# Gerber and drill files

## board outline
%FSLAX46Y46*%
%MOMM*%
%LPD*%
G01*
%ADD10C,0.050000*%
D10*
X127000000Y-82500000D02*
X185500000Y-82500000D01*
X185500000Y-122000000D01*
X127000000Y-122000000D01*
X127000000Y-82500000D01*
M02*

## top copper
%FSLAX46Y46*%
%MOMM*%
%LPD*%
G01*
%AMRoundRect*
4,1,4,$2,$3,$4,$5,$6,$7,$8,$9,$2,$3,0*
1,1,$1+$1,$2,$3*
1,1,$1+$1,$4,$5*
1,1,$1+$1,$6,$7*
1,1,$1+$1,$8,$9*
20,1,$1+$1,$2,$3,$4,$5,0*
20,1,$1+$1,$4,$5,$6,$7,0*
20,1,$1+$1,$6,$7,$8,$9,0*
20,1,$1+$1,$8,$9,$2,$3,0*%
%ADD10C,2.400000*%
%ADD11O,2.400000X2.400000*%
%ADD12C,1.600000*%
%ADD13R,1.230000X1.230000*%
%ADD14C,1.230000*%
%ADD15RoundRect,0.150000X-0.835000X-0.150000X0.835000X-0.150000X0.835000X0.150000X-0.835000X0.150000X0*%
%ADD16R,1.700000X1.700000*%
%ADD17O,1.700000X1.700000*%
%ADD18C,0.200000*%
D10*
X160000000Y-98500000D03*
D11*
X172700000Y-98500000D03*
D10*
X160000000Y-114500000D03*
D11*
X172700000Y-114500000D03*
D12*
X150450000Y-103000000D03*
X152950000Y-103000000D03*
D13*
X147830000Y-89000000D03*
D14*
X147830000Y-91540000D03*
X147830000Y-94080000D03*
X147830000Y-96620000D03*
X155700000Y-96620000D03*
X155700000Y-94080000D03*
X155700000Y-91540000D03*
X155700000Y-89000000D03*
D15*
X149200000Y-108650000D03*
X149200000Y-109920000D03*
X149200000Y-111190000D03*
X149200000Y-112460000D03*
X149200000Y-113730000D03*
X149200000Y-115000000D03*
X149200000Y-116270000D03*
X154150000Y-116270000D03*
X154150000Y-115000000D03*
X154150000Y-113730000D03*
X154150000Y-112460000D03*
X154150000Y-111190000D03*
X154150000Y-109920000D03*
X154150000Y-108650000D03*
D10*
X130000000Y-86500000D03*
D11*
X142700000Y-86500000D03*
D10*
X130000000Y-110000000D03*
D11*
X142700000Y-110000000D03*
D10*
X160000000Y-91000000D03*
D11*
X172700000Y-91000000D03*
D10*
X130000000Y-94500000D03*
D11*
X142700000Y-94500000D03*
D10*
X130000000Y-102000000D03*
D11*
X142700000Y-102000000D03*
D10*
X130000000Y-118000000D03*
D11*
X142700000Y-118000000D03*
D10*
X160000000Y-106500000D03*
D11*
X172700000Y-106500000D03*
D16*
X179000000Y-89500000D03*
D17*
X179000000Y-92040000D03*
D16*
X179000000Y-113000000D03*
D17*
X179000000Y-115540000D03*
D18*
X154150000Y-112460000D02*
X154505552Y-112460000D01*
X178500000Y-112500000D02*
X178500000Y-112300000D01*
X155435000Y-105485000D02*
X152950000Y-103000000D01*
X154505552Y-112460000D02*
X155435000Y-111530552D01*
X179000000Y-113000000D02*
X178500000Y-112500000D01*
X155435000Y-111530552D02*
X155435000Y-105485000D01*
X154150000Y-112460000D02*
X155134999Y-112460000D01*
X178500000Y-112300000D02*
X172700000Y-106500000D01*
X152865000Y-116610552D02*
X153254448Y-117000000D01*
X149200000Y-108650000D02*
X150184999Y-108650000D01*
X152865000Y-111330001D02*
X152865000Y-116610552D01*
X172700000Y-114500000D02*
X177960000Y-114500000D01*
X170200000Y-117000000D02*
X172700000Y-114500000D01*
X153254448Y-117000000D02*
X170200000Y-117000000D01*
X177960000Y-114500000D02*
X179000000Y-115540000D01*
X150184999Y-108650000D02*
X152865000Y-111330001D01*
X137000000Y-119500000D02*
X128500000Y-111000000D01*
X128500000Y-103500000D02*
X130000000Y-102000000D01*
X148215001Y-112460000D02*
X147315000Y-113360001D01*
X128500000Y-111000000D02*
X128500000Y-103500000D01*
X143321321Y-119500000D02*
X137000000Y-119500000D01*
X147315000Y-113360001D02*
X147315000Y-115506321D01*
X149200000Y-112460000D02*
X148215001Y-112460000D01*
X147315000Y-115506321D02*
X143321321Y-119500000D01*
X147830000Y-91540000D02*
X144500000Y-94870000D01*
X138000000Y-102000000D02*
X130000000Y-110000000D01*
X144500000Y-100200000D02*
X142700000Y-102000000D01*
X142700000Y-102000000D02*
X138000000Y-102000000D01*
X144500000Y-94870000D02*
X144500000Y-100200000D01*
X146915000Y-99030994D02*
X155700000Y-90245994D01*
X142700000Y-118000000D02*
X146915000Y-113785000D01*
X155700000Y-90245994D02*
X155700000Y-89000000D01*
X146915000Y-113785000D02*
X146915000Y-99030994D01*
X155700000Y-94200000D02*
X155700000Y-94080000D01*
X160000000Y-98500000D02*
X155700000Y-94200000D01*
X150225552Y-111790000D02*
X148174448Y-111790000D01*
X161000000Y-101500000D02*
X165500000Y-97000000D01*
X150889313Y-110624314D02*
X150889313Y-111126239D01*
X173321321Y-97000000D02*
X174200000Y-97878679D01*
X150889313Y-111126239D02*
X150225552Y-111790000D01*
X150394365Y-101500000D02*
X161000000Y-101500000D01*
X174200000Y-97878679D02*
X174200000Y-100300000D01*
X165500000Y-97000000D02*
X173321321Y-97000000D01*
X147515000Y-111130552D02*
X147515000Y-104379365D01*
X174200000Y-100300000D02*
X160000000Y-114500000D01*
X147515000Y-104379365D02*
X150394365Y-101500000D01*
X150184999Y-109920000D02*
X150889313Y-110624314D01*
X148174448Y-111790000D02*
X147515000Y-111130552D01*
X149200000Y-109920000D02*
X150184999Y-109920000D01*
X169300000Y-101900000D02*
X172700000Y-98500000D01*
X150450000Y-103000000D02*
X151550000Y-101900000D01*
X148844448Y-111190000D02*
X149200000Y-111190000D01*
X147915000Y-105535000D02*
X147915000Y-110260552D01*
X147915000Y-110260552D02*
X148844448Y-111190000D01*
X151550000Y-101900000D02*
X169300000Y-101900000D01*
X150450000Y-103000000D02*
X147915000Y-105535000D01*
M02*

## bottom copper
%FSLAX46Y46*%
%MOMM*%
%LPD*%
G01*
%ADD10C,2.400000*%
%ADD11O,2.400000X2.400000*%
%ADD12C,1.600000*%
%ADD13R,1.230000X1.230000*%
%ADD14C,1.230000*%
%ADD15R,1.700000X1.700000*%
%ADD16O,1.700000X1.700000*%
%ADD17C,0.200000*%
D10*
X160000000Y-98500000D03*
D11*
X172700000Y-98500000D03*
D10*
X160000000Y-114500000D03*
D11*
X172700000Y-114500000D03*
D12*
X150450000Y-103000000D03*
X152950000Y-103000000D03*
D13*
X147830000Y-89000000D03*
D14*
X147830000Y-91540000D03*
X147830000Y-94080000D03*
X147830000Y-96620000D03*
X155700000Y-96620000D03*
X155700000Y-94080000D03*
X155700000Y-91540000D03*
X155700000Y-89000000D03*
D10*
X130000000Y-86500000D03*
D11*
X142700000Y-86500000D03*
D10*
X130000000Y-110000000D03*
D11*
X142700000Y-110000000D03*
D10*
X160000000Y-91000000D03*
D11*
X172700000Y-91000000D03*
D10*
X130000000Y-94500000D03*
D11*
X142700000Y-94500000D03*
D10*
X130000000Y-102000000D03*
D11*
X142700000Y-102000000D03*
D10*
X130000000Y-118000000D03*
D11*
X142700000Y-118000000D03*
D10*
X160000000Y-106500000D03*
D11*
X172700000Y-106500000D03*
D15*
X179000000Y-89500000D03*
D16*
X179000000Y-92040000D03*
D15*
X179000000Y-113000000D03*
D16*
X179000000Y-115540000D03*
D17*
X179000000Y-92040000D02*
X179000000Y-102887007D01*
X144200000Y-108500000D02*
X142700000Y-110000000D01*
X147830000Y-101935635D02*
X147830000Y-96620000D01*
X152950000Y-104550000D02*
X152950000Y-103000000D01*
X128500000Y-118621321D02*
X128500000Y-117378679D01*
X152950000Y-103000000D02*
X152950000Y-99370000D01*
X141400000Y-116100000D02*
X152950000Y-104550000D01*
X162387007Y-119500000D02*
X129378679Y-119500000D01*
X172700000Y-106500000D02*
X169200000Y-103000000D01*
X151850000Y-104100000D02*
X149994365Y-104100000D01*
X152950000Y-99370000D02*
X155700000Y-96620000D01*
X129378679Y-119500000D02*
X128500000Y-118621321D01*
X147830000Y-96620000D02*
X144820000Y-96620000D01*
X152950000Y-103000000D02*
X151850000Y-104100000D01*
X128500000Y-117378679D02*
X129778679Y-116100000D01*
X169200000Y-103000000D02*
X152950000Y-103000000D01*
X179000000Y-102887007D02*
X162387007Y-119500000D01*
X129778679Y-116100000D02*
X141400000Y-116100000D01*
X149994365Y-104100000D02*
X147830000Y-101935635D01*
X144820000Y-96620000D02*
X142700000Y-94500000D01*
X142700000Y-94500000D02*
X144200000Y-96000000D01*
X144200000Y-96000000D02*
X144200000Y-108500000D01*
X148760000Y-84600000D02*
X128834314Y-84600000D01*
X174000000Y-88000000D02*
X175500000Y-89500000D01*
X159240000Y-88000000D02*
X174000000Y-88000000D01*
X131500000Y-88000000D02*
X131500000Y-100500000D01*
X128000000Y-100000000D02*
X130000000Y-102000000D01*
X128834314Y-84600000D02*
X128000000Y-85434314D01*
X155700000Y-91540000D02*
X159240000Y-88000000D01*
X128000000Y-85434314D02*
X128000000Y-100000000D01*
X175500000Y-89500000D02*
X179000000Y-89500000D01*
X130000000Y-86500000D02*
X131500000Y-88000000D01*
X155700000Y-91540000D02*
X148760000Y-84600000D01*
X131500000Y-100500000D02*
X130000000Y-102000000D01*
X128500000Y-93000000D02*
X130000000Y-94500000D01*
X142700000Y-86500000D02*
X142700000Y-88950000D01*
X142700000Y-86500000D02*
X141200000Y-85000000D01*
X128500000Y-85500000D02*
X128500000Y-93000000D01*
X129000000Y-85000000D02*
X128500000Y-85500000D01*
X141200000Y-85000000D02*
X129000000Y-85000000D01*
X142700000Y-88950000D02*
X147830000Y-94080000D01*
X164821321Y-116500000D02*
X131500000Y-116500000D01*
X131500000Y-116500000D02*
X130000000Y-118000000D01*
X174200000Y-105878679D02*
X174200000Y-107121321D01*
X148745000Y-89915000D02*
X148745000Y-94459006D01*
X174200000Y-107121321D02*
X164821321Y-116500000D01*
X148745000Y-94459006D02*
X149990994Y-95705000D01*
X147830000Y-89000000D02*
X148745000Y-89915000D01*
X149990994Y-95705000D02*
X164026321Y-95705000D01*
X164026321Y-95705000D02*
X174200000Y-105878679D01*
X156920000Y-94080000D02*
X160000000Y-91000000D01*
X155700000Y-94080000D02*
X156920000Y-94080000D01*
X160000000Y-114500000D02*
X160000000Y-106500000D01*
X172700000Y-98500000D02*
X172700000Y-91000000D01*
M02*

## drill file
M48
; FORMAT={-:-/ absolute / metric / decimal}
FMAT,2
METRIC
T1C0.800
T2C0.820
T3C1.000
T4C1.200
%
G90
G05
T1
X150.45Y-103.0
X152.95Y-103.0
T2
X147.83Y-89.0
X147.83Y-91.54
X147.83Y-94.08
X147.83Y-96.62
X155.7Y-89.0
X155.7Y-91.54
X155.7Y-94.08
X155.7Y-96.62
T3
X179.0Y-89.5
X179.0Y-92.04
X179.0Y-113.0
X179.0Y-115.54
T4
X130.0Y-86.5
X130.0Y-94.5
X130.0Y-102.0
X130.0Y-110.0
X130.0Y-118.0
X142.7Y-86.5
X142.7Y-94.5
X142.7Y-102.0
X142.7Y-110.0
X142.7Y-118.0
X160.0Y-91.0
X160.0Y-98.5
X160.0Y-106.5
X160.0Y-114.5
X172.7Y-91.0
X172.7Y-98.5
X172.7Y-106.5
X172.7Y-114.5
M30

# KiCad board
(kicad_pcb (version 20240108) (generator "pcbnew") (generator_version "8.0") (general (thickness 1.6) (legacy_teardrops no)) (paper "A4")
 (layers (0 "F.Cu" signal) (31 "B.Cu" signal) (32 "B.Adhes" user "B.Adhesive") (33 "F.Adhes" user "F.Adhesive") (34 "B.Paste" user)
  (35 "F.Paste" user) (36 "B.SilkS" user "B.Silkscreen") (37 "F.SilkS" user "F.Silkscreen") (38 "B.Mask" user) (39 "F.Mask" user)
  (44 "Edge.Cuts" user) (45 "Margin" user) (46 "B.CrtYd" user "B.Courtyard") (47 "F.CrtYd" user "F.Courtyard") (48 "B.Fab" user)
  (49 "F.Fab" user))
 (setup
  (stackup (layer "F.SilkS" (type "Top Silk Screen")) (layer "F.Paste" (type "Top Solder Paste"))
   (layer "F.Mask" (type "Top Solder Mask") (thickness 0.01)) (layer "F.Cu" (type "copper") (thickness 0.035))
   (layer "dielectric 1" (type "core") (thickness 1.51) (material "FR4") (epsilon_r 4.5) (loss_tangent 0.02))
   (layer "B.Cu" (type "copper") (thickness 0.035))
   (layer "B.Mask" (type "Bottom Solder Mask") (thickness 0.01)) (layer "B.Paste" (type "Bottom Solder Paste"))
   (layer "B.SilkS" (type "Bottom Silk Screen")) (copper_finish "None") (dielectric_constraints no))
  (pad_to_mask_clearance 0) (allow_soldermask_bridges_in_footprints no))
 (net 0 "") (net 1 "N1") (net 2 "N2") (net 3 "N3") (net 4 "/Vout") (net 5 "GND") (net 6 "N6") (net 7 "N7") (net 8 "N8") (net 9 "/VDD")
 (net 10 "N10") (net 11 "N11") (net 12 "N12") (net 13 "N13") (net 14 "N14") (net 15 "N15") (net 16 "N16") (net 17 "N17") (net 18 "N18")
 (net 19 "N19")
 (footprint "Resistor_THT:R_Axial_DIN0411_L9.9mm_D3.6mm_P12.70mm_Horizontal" (layer "F.Cu") (at 160 98.5)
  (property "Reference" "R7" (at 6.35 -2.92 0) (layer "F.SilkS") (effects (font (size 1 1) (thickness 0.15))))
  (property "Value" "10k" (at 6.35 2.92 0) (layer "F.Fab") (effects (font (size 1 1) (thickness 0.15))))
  (pad "1" thru_hole circle (at 0 0) (size 2.4 2.4) (drill 1.2) (layers "*.Cu" "*.Mask") (remove_unused_layers no) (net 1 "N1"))
  (pad "2" thru_hole oval (at 12.7 0) (size 2.4 2.4) (drill 1.2) (layers "*.Cu" "*.Mask") (remove_unused_layers no) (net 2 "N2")))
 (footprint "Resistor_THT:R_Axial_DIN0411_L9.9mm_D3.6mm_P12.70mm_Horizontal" (layer "F.Cu") (at 160 114.5)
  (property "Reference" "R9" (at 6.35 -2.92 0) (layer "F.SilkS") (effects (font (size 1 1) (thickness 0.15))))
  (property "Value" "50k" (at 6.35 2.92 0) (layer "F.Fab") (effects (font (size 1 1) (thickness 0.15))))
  (pad "1" thru_hole circle (at 0 0) (size 2.4 2.4) (drill 1.2) (layers "*.Cu" "*.Mask") (remove_unused_layers no) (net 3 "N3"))
  (pad "2" thru_hole oval (at 12.7 0) (size 2.4 2.4) (drill 1.2) (layers "*.Cu" "*.Mask") (remove_unused_layers no) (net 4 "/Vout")))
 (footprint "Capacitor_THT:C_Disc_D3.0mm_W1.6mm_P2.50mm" (layer "F.Cu") (at 150.45 103)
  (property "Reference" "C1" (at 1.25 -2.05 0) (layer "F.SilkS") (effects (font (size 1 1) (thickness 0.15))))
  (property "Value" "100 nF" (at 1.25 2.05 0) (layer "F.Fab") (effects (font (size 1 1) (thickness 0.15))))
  (pad "1" thru_hole circle (at 0 0) (size 1.6 1.6) (drill 0.8) (layers "*.Cu" "*.Mask") (remove_unused_layers no) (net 2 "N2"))
  (pad "2" thru_hole circle (at 2.5 0) (size 1.6 1.6) (drill 0.8) (layers "*.Cu" "*.Mask") (remove_unused_layers no) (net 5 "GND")))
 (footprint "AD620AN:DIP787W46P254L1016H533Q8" (layer "F.Cu") (at 151.765 92.81)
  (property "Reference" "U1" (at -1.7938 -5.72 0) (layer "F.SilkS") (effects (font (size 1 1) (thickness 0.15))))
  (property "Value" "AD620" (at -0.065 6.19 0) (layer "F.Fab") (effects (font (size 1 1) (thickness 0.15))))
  (pad "1" thru_hole rect (at -3.935 -3.81) (size 1.23 1.23) (drill 0.82) (layers "*.Cu" "*.Mask") (remove_unused_layers no) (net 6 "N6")
   (solder_mask_margin 0.102))
  (pad "2" thru_hole circle (at -3.935 -1.27) (size 1.23 1.23) (drill 0.82) (layers "*.Cu" "*.Mask") (remove_unused_layers no) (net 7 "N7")
   (solder_mask_margin 0.102))
  (pad "3" thru_hole circle (at -3.935 1.27) (size 1.23 1.23) (drill 0.82) (layers "*.Cu" "*.Mask") (remove_unused_layers no) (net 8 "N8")
   (solder_mask_margin 0.102))
  (pad "4" thru_hole circle (at -3.935 3.81) (size 1.23 1.23) (drill 0.82) (layers "*.Cu" "*.Mask") (remove_unused_layers no) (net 5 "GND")
   (solder_mask_margin 0.102))
  (pad "5" thru_hole circle (at 3.935 3.81) (size 1.23 1.23) (drill 0.82) (layers "*.Cu" "*.Mask") (remove_unused_layers no) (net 5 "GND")
   (solder_mask_margin 0.102))
  (pad "6" thru_hole circle (at 3.935 1.27) (size 1.23 1.23) (drill 0.82) (layers "*.Cu" "*.Mask") (remove_unused_layers no) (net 1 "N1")
   (solder_mask_margin 0.102))
  (pad "7" thru_hole circle (at 3.935 -1.27) (size 1.23 1.23) (drill 0.82) (layers "*.Cu" "*.Mask") (remove_unused_layers no) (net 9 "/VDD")
   (solder_mask_margin 0.102))
  (pad "8" thru_hole circle (at 3.935 -3.81) (size 1.23 1.23) (drill 0.82) (layers "*.Cu" "*.Mask") (remove_unused_layers no) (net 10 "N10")
   (solder_mask_margin 0.102)))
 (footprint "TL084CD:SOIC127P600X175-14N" (layer "F.Cu") (at 151.675 112.46)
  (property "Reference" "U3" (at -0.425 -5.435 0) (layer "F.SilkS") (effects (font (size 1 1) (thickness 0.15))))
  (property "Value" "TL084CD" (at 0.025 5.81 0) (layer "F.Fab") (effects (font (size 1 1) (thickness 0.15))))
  (pad "1" smd roundrect (at -2.475 -3.81) (size 1.97 0.6) (layers "F.Cu" "F.Paste" "F.Mask") (roundrect_rratio 0.25) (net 4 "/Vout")
   (solder_mask_margin 0.102))
  (pad "2" smd roundrect (at -2.475 -2.54) (size 1.97 0.6) (layers "F.Cu" "F.Paste" "F.Mask") (roundrect_rratio 0.25) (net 3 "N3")
   (solder_mask_margin 0.102))
  (pad "3" smd roundrect (at -2.475 -1.27) (size 1.97 0.6) (layers "F.Cu" "F.Paste" "F.Mask") (roundrect_rratio 0.25) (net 2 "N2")
   (solder_mask_margin 0.102))
  (pad "4" smd roundrect (at -2.475 0) (size 1.97 0.6) (layers "F.Cu" "F.Paste" "F.Mask") (roundrect_rratio 0.25) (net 9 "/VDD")
   (solder_mask_margin 0.102))
  (pad "5" smd roundrect (at -2.475 1.27) (size 1.97 0.6) (layers "F.Cu" "F.Paste" "F.Mask") (roundrect_rratio 0.25) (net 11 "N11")
   (solder_mask_margin 0.102))
  (pad "6" smd roundrect (at -2.475 2.54) (size 1.97 0.6) (layers "F.Cu" "F.Paste" "F.Mask") (roundrect_rratio 0.25) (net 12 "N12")
   (solder_mask_margin 0.102))
  (pad "7" smd roundrect (at -2.475 3.81) (size 1.97 0.6) (layers "F.Cu" "F.Paste" "F.Mask") (roundrect_rratio 0.25) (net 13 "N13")
   (solder_mask_margin 0.102))
  (pad "8" smd roundrect (at 2.475 3.81) (size 1.97 0.6) (layers "F.Cu" "F.Paste" "F.Mask") (roundrect_rratio 0.25) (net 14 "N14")
   (solder_mask_margin 0.102))
  (pad "9" smd roundrect (at 2.475 2.54) (size 1.97 0.6) (layers "F.Cu" "F.Paste" "F.Mask") (roundrect_rratio 0.25) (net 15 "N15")
   (solder_mask_margin 0.102))
  (pad "10" smd roundrect (at 2.475 1.27) (size 1.97 0.6) (layers "F.Cu" "F.Paste" "F.Mask") (roundrect_rratio 0.25) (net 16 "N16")
   (solder_mask_margin 0.102))
  (pad "11" smd roundrect (at 2.475 0) (size 1.97 0.6) (layers "F.Cu" "F.Paste" "F.Mask") (roundrect_rratio 0.25) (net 5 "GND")
   (solder_mask_margin 0.102))
  (pad "12" smd roundrect (at 2.475 -1.27) (size 1.97 0.6) (layers "F.Cu" "F.Paste" "F.Mask") (roundrect_rratio 0.25) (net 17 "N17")
   (solder_mask_margin 0.102))
  (pad "13" smd roundrect (at 2.475 -2.54) (size 1.97 0.6) (layers "F.Cu" "F.Paste" "F.Mask") (roundrect_rratio 0.25) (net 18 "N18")
   (solder_mask_margin 0.102))
  (pad "14" smd roundrect (at 2.475 -3.81) (size 1.97 0.6) (layers "F.Cu" "F.Paste" "F.Mask") (roundrect_rratio 0.25) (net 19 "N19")
   (solder_mask_margin 0.102)))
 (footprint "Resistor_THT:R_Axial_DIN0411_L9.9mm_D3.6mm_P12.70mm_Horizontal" (layer "F.Cu") (at 130 86.5)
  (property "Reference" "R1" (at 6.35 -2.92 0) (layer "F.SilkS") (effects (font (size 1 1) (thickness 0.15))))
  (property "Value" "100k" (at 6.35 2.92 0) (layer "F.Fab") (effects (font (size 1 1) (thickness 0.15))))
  (pad "1" thru_hole circle (at 0 0) (size 2.4 2.4) (drill 1.2) (layers "*.Cu" "*.Mask") (remove_unused_layers no) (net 9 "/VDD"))
  (pad "2" thru_hole oval (at 12.7 0) (size 2.4 2.4) (drill 1.2) (layers "*.Cu" "*.Mask") (remove_unused_layers no) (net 8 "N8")))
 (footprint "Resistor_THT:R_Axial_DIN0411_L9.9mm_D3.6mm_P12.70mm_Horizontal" (layer "F.Cu") (at 130 110)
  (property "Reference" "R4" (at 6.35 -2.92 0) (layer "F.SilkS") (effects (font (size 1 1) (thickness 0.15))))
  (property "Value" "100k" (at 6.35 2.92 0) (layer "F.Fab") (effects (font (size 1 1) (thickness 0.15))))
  (pad "1" thru_hole circle (at 0 0) (size 2.4 2.4) (drill 1.2) (layers "*.Cu" "*.Mask") (remove_unused_layers no) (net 7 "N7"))
  (pad "2" thru_hole oval (at 12.7 0) (size 2.4 2.4) (drill 1.2) (layers "*.Cu" "*.Mask") (remove_unused_layers no) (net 5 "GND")))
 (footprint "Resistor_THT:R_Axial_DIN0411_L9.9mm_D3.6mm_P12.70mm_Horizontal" (layer "F.Cu") (at 160 91)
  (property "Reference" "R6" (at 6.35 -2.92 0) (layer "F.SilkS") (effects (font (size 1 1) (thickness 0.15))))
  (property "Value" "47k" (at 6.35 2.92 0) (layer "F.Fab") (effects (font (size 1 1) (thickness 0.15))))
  (pad "1" thru_hole circle (at 0 0) (size 2.4 2.4) (drill 1.2) (layers "*.Cu" "*.Mask") (remove_unused_layers no) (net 1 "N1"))
  (pad "2" thru_hole oval (at 12.7 0) (size 2.4 2.4) (drill 1.2) (layers "*.Cu" "*.Mask") (remove_unused_layers no) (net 2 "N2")))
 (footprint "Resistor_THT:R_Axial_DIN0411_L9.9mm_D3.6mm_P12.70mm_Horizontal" (layer "F.Cu") (at 130 94.5)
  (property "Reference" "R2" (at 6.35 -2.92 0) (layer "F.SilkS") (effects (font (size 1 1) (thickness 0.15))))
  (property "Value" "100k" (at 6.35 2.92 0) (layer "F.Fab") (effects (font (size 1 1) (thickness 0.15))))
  (pad "1" thru_hole circle (at 0 0) (size 2.4 2.4) (drill 1.2) (layers "*.Cu" "*.Mask") (remove_unused_layers no) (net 8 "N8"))
  (pad "2" thru_hole oval (at 12.7 0) (size 2.4 2.4) (drill 1.2) (layers "*.Cu" "*.Mask") (remove_unused_layers no) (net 5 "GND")))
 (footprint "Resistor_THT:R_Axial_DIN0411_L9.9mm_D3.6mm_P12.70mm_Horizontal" (layer "F.Cu") (at 130 102)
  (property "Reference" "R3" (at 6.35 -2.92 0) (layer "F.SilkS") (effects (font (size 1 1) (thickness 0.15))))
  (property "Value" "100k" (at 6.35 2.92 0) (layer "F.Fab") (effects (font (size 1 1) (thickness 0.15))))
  (pad "1" thru_hole circle (at 0 0) (size 2.4 2.4) (drill 1.2) (layers "*.Cu" "*.Mask") (remove_unused_layers no) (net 9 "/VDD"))
  (pad "2" thru_hole oval (at 12.7 0) (size 2.4 2.4) (drill 1.2) (layers "*.Cu" "*.Mask") (remove_unused_layers no) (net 7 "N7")))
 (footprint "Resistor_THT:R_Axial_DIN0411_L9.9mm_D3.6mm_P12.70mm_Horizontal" (layer "F.Cu") (at 130 118)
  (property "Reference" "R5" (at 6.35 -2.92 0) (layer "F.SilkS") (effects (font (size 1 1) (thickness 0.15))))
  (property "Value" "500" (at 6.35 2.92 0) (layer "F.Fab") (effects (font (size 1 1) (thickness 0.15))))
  (pad "1" thru_hole circle (at 0 0) (size 2.4 2.4) (drill 1.2) (layers "*.Cu" "*.Mask") (remove_unused_layers no) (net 6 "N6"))
  (pad "2" thru_hole oval (at 12.7 0) (size 2.4 2.4) (drill 1.2) (layers "*.Cu" "*.Mask") (remove_unused_layers no) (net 10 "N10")))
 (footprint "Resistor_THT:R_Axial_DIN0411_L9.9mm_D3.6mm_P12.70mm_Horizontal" (layer "F.Cu") (at 160 106.5)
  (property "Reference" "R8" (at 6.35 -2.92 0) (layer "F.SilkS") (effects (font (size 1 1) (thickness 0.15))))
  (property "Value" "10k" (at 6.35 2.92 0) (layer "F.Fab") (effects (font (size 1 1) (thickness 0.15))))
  (pad "1" thru_hole circle (at 0 0) (size 2.4 2.4) (drill 1.2) (layers "*.Cu" "*.Mask") (remove_unused_layers no) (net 3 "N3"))
  (pad "2" thru_hole oval (at 12.7 0) (size 2.4 2.4) (drill 1.2) (layers "*.Cu" "*.Mask") (remove_unused_layers no) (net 5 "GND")))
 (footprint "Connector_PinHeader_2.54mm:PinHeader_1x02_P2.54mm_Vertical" (layer "F.Cu") (at 179 89.5)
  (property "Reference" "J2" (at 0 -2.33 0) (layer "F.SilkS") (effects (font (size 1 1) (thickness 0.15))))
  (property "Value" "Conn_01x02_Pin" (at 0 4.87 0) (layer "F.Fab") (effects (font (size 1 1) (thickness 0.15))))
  (pad "1" thru_hole rect (at 0 0) (size 1.7 1.7) (drill 1) (layers "*.Cu" "*.Mask") (remove_unused_layers no) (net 9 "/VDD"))
  (pad "2" thru_hole oval (at 0 2.54) (size 1.7 1.7) (drill 1) (layers "*.Cu" "*.Mask") (remove_unused_layers no) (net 5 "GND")))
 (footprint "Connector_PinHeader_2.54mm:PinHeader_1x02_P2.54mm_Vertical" (layer "F.Cu") (at 179 113)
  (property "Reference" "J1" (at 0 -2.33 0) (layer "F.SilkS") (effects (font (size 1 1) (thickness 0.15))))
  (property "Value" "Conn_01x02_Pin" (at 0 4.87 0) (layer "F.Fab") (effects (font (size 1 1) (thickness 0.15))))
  (pad "1" thru_hole rect (at 0 0) (size 1.7 1.7) (drill 1) (layers "*.Cu" "*.Mask") (remove_unused_layers no) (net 5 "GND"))
  (pad "2" thru_hole oval (at 0 2.54) (size 1.7 1.7) (drill 1) (layers "*.Cu" "*.Mask") (remove_unused_layers no) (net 4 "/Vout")))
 (gr_rect (start 127 82.5) (end 185.5 122) (stroke (width 0.05) (type default)) (fill none) (layer "Edge.Cuts"))
 (segment (start 154.15 112.46) (end 154.505552 112.46) (width 0.2) (layer "F.Cu") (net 5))
 (segment (start 178.5 112.5) (end 178.5 112.3) (width 0.2) (layer "F.Cu") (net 5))
 (segment (start 155.435 105.485) (end 152.95 103) (width 0.2) (layer "F.Cu") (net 5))
 (segment (start 154.505552 112.46) (end 155.435 111.530552) (width 0.2) (layer "F.Cu") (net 5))
 (segment (start 179 113) (end 178.5 112.5) (width 0.2) (layer "F.Cu") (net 5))
 (segment (start 155.435 111.530552) (end 155.435 105.485) (width 0.2) (layer "F.Cu") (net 5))
 (segment (start 154.15 112.46) (end 155.134999 112.46) (width 0.2) (layer "F.Cu") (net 5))
 (segment (start 178.5 112.3) (end 172.7 106.5) (width 0.2) (layer "F.Cu") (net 5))
 (segment (start 179 92.04) (end 179 102.887007) (width 0.2) (layer "B.Cu") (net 5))
 (segment (start 144.2 108.5) (end 142.7 110) (width 0.2) (layer "B.Cu") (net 5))
 (segment (start 147.83 101.935635) (end 147.83 96.62) (width 0.2) (layer "B.Cu") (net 5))
 (segment (start 152.95 104.55) (end 152.95 103) (width 0.2) (layer "B.Cu") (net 5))
 (segment (start 128.5 118.621321) (end 128.5 117.378679) (width 0.2) (layer "B.Cu") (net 5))
 (segment (start 152.95 103) (end 152.95 99.37) (width 0.2) (layer "B.Cu") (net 5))
 (segment (start 141.4 116.1) (end 152.95 104.55) (width 0.2) (layer "B.Cu") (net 5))
 (segment (start 162.387007 119.5) (end 129.378679 119.5) (width 0.2) (layer "B.Cu") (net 5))
 (segment (start 172.7 106.5) (end 169.2 103) (width 0.2) (layer "B.Cu") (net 5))
 (segment (start 151.85 104.1) (end 149.994365 104.1) (width 0.2) (layer "B.Cu") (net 5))
 (segment (start 152.95 99.37) (end 155.7 96.62) (width 0.2) (layer "B.Cu") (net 5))
 (segment (start 129.378679 119.5) (end 128.5 118.621321) (width 0.2) (layer "B.Cu") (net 5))
 (segment (start 147.83 96.62) (end 144.82 96.62) (width 0.2) (layer "B.Cu") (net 5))
 (segment (start 152.95 103) (end 151.85 104.1) (width 0.2) (layer "B.Cu") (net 5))
 (segment (start 128.5 117.378679) (end 129.778679 116.1) (width 0.2) (layer "B.Cu") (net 5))
 (segment (start 169.2 103) (end 152.95 103) (width 0.2) (layer "B.Cu") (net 5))
 (segment (start 179 102.887007) (end 162.387007 119.5) (width 0.2) (layer "B.Cu") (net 5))
 (segment (start 129.778679 116.1) (end 141.4 116.1) (width 0.2) (layer "B.Cu") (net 5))
 (segment (start 149.994365 104.1) (end 147.83 101.935635) (width 0.2) (layer "B.Cu") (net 5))
 (segment (start 144.82 96.62) (end 142.7 94.5) (width 0.2) (layer "B.Cu") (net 5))
 (segment (start 142.7 94.5) (end 144.2 96) (width 0.2) (layer "B.Cu") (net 5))
 (segment (start 144.2 96) (end 144.2 108.5) (width 0.2) (layer "B.Cu") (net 5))
 (segment (start 152.865 116.610552) (end 153.254448 117) (width 0.2) (layer "F.Cu") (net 4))
 (segment (start 149.2 108.65) (end 150.184999 108.65) (width 0.2) (layer "F.Cu") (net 4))
 (segment (start 152.865 111.330001) (end 152.865 116.610552) (width 0.2) (layer "F.Cu") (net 4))
 (segment (start 172.7 114.5) (end 177.96 114.5) (width 0.2) (layer "F.Cu") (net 4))
 (segment (start 170.2 117) (end 172.7 114.5) (width 0.2) (layer "F.Cu") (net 4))
 (segment (start 153.254448 117) (end 170.2 117) (width 0.2) (layer "F.Cu") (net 4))
 (segment (start 177.96 114.5) (end 179 115.54) (width 0.2) (layer "F.Cu") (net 4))
 (segment (start 150.184999 108.65) (end 152.865 111.330001) (width 0.2) (layer "F.Cu") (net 4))
 (segment (start 137 119.5) (end 128.5 111) (width 0.2) (layer "F.Cu") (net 9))
 (segment (start 128.5 103.5) (end 130 102) (width 0.2) (layer "F.Cu") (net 9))
 (segment (start 148.215001 112.46) (end 147.315 113.360001) (width 0.2) (layer "F.Cu") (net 9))
 (segment (start 128.5 111) (end 128.5 103.5) (width 0.2) (layer "F.Cu") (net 9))
 (segment (start 143.321321 119.5) (end 137 119.5) (width 0.2) (layer "F.Cu") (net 9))
 (segment (start 147.315 113.360001) (end 147.315 115.506321) (width 0.2) (layer "F.Cu") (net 9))
 (segment (start 149.2 112.46) (end 148.215001 112.46) (width 0.2) (layer "F.Cu") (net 9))
 (segment (start 147.315 115.506321) (end 143.321321 119.5) (width 0.2) (layer "F.Cu") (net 9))
 (segment (start 148.76 84.6) (end 128.834314 84.6) (width 0.2) (layer "B.Cu") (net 9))
 (segment (start 174 88) (end 175.5 89.5) (width 0.2) (layer "B.Cu") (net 9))
 (segment (start 159.24 88) (end 174 88) (width 0.2) (layer "B.Cu") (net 9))
 (segment (start 131.5 88) (end 131.5 100.5) (width 0.2) (layer "B.Cu") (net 9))
 (segment (start 128 100) (end 130 102) (width 0.2) (layer "B.Cu") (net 9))
 (segment (start 128.834314 84.6) (end 128 85.434314) (width 0.2) (layer "B.Cu") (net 9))
 (segment (start 155.7 91.54) (end 159.24 88) (width 0.2) (layer "B.Cu") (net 9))
 (segment (start 128 85.434314) (end 128 100) (width 0.2) (layer "B.Cu") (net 9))
 (segment (start 175.5 89.5) (end 179 89.5) (width 0.2) (layer "B.Cu") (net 9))
 (segment (start 130 86.5) (end 131.5 88) (width 0.2) (layer "B.Cu") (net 9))
 (segment (start 155.7 91.54) (end 148.76 84.6) (width 0.2) (layer "B.Cu") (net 9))
 (segment (start 131.5 100.5) (end 130 102) (width 0.2) (layer "B.Cu") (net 9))
 (segment (start 128.5 93) (end 130 94.5) (width 0.2) (layer "B.Cu") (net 8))
 (segment (start 142.7 86.5) (end 142.7 88.95) (width 0.2) (layer "B.Cu") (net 8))
 (segment (start 142.7 86.5) (end 141.2 85) (width 0.2) (layer "B.Cu") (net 8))
 (segment (start 128.5 85.5) (end 128.5 93) (width 0.2) (layer "B.Cu") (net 8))
 (segment (start 129 85) (end 128.5 85.5) (width 0.2) (layer "B.Cu") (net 8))
 (segment (start 141.2 85) (end 129 85) (width 0.2) (layer "B.Cu") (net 8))
 (segment (start 142.7 88.95) (end 147.83 94.08) (width 0.2) (layer "B.Cu") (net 8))
 (segment (start 147.83 91.54) (end 144.5 94.87) (width 0.2) (layer "F.Cu") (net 7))
 (segment (start 138 102) (end 130 110) (width 0.2) (layer "F.Cu") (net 7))
 (segment (start 144.5 100.2) (end 142.7 102) (width 0.2) (layer "F.Cu") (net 7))
 (segment (start 142.7 102) (end 138 102) (width 0.2) (layer "F.Cu") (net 7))
 (segment (start 144.5 94.87) (end 144.5 100.2) (width 0.2) (layer "F.Cu") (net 7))
 (segment (start 164.821321 116.5) (end 131.5 116.5) (width 0.2) (layer "B.Cu") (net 6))
 (segment (start 131.5 116.5) (end 130 118) (width 0.2) (layer "B.Cu") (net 6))
 (segment (start 174.2 105.878679) (end 174.2 107.121321) (width 0.2) (layer "B.Cu") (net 6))
 (segment (start 148.745 89.915) (end 148.745 94.459006) (width 0.2) (layer "B.Cu") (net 6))
 (segment (start 174.2 107.121321) (end 164.821321 116.5) (width 0.2) (layer "B.Cu") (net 6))
 (segment (start 148.745 94.459006) (end 149.990994 95.705) (width 0.2) (layer "B.Cu") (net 6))
 (segment (start 147.83 89) (end 148.745 89.915) (width 0.2) (layer "B.Cu") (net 6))
 (segment (start 149.990994 95.705) (end 164.026321 95.705) (width 0.2) (layer "B.Cu") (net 6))
 (segment (start 164.026321 95.705) (end 174.2 105.878679) (width 0.2) (layer "B.Cu") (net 6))
 (segment (start 146.915 99.030994) (end 155.7 90.245994) (width 0.2) (layer "F.Cu") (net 10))
 (segment (start 142.7 118) (end 146.915 113.785) (width 0.2) (layer "F.Cu") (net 10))
 (segment (start 155.7 90.245994) (end 155.7 89) (width 0.2) (layer "F.Cu") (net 10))
 (segment (start 146.915 113.785) (end 146.915 99.030994) (width 0.2) (layer "F.Cu") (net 10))
 (segment (start 155.7 94.2) (end 155.7 94.08) (width 0.2) (layer "F.Cu") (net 1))
 (segment (start 160 98.5) (end 155.7 94.2) (width 0.2) (layer "F.Cu") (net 1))
 (segment (start 156.92 94.08) (end 160 91) (width 0.2) (layer "B.Cu") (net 1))
 (segment (start 155.7 94.08) (end 156.92 94.08) (width 0.2) (layer "B.Cu") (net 1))
 (segment (start 150.225552 111.79) (end 148.174448 111.79) (width 0.2) (layer "F.Cu") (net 3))
 (segment (start 161 101.5) (end 165.5 97) (width 0.2) (layer "F.Cu") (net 3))
 (segment (start 150.889313 110.624314) (end 150.889313 111.126239) (width 0.2) (layer "F.Cu") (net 3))
 (segment (start 173.321321 97) (end 174.2 97.878679) (width 0.2) (layer "F.Cu") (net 3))
 (segment (start 150.889313 111.126239) (end 150.225552 111.79) (width 0.2) (layer "F.Cu") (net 3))
 (segment (start 150.394365 101.5) (end 161 101.5) (width 0.2) (layer "F.Cu") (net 3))
 (segment (start 174.2 97.878679) (end 174.2 100.3) (width 0.2) (layer "F.Cu") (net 3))
 (segment (start 165.5 97) (end 173.321321 97) (width 0.2) (layer "F.Cu") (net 3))
 (segment (start 147.515 111.130552) (end 147.515 104.379365) (width 0.2) (layer "F.Cu") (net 3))
 (segment (start 174.2 100.3) (end 160 114.5) (width 0.2) (layer "F.Cu") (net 3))
 (segment (start 147.515 104.379365) (end 150.394365 101.5) (width 0.2) (layer "F.Cu") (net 3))
 (segment (start 150.184999 109.92) (end 150.889313 110.624314) (width 0.2) (layer "F.Cu") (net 3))
 (segment (start 148.174448 111.79) (end 147.515 111.130552) (width 0.2) (layer "F.Cu") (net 3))
 (segment (start 149.2 109.92) (end 150.184999 109.92) (width 0.2) (layer "F.Cu") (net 3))
 (segment (start 160 114.5) (end 160 106.5) (width 0.2) (layer "B.Cu") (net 3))
 (segment (start 169.3 101.9) (end 172.7 98.5) (width 0.2) (layer "F.Cu") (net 2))
 (segment (start 150.45 103) (end 151.55 101.9) (width 0.2) (layer "F.Cu") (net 2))
 (segment (start 148.844448 111.19) (end 149.2 111.19) (width 0.2) (layer "F.Cu") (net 2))
 (segment (start 147.915 105.535) (end 147.915 110.260552) (width 0.2) (layer "F.Cu") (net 2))
 (segment (start 147.915 110.260552) (end 148.844448 111.19) (width 0.2) (layer "F.Cu") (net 2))
 (segment (start 151.55 101.9) (end 169.3 101.9) (width 0.2) (layer "F.Cu") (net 2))
 (segment (start 150.45 103) (end 147.915 105.535) (width 0.2) (layer "F.Cu") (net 2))
 (segment (start 172.7 98.5) (end 172.7 91) (width 0.2) (layer "B.Cu") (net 2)))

